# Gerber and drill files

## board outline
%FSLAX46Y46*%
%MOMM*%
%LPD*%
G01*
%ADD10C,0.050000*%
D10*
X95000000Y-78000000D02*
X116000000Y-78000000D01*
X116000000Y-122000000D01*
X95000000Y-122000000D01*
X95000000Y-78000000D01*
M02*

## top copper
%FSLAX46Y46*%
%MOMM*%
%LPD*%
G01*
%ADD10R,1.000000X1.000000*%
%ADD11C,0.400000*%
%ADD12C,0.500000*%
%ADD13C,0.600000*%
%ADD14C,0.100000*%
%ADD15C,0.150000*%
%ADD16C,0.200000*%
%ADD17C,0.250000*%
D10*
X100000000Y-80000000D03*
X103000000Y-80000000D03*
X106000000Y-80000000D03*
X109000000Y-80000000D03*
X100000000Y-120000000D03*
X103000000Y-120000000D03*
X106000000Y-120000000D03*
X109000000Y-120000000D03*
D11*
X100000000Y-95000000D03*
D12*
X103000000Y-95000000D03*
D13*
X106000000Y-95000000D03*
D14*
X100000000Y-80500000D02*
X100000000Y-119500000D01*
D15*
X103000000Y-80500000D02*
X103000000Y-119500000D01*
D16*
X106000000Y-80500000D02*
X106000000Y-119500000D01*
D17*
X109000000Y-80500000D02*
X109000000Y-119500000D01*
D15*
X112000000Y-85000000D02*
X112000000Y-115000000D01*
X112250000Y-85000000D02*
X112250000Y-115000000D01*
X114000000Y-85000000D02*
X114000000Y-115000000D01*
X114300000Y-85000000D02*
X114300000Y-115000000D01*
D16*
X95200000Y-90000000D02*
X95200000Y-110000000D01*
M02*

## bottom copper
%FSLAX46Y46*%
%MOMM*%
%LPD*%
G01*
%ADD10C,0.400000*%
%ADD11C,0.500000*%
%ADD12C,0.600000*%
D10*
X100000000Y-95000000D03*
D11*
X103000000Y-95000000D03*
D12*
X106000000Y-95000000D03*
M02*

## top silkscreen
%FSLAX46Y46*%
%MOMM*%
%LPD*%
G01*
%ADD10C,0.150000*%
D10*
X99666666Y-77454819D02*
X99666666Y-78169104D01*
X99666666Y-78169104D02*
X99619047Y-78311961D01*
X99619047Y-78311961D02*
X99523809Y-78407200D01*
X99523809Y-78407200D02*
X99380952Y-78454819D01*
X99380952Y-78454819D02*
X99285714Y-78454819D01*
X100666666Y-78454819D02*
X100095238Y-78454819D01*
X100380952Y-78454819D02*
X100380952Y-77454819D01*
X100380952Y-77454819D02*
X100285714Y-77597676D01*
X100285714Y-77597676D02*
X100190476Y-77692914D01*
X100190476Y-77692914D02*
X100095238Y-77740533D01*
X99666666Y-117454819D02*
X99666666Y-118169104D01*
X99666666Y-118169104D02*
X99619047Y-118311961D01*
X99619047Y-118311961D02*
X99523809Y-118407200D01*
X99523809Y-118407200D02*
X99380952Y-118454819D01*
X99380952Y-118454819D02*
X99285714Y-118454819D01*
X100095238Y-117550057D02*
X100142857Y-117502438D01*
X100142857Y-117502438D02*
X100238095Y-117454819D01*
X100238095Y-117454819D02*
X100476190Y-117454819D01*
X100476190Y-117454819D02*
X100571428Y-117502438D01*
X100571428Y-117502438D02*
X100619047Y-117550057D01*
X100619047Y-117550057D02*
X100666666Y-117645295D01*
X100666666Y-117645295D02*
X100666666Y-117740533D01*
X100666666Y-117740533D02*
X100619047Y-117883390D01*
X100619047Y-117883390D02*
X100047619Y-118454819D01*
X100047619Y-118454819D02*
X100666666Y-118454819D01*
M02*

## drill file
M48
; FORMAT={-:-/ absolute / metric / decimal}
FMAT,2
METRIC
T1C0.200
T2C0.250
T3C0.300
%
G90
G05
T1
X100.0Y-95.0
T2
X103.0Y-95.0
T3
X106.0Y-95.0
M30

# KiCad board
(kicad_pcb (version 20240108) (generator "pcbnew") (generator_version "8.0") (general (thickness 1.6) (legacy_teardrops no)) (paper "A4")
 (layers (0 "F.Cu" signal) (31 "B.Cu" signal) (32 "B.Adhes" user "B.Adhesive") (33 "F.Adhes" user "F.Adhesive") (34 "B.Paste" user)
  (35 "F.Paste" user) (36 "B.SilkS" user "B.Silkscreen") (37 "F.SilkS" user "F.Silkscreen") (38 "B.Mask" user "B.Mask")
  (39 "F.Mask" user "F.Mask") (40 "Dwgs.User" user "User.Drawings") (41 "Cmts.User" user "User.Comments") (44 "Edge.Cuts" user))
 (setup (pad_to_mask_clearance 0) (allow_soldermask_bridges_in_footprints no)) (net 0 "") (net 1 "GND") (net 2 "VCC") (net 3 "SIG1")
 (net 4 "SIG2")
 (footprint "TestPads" (layer "F.Cu") (at 100 80) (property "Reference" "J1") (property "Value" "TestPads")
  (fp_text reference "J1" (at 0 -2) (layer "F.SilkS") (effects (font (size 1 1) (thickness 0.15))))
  (pad "1" smd rect (at 0 0) (size 1 1) (layers "F.Cu" "F.Paste" "F.Mask") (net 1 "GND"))
  (pad "2" smd rect (at 3 0) (size 1 1) (layers "F.Cu" "F.Paste" "F.Mask") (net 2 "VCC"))
  (pad "3" smd rect (at 6 0) (size 1 1) (layers "F.Cu" "F.Paste" "F.Mask") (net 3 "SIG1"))
  (pad "4" smd rect (at 9 0) (size 1 1) (layers "F.Cu" "F.Paste" "F.Mask") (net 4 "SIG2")))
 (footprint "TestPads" (layer "F.Cu") (at 100 120) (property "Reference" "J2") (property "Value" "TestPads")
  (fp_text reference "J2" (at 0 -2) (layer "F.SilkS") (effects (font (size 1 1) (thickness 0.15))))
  (pad "1" smd rect (at 0 0) (size 1 1) (layers "F.Cu" "F.Paste" "F.Mask") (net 1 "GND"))
  (pad "2" smd rect (at 3 0) (size 1 1) (layers "F.Cu" "F.Paste" "F.Mask") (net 2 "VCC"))
  (pad "3" smd rect (at 6 0) (size 1 1) (layers "F.Cu" "F.Paste" "F.Mask") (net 3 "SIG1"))
  (pad "4" smd rect (at 9 0) (size 1 1) (layers "F.Cu" "F.Paste" "F.Mask") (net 4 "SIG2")))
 (segment (start 100 80.5) (end 100 119.5) (width 0.1) (layer "F.Cu") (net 1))
 (segment (start 103 80.5) (end 103 119.5) (width 0.15) (layer "F.Cu") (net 2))
 (segment (start 106 80.5) (end 106 119.5) (width 0.2) (layer "F.Cu") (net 3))
 (segment (start 109 80.5) (end 109 119.5) (width 0.25) (layer "F.Cu") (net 4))
 (via (at 100 95) (size 0.4) (drill 0.2) (layers "F.Cu" "B.Cu") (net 1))
 (via (at 103 95) (size 0.5) (drill 0.25) (layers "F.Cu" "B.Cu") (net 2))
 (via (at 106 95) (size 0.6) (drill 0.3) (layers "F.Cu" "B.Cu") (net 3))
 (segment (start 112 85) (end 112 115) (width 0.15) (layer "F.Cu") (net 3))
 (segment (start 112.25 85) (end 112.25 115) (width 0.15) (layer "F.Cu") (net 4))
 (segment (start 114 85) (end 114 115) (width 0.15) (layer "F.Cu") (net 1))
 (segment (start 114.3 85) (end 114.3 115) (width 0.15) (layer "F.Cu") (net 2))
 (segment (start 95.2 90) (end 95.2 110) (width 0.2) (layer "F.Cu") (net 3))
 (gr_rect (start 95 78) (end 116 122) (stroke (width 0.05) (type default)) (fill none) (layer "Edge.Cuts")))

